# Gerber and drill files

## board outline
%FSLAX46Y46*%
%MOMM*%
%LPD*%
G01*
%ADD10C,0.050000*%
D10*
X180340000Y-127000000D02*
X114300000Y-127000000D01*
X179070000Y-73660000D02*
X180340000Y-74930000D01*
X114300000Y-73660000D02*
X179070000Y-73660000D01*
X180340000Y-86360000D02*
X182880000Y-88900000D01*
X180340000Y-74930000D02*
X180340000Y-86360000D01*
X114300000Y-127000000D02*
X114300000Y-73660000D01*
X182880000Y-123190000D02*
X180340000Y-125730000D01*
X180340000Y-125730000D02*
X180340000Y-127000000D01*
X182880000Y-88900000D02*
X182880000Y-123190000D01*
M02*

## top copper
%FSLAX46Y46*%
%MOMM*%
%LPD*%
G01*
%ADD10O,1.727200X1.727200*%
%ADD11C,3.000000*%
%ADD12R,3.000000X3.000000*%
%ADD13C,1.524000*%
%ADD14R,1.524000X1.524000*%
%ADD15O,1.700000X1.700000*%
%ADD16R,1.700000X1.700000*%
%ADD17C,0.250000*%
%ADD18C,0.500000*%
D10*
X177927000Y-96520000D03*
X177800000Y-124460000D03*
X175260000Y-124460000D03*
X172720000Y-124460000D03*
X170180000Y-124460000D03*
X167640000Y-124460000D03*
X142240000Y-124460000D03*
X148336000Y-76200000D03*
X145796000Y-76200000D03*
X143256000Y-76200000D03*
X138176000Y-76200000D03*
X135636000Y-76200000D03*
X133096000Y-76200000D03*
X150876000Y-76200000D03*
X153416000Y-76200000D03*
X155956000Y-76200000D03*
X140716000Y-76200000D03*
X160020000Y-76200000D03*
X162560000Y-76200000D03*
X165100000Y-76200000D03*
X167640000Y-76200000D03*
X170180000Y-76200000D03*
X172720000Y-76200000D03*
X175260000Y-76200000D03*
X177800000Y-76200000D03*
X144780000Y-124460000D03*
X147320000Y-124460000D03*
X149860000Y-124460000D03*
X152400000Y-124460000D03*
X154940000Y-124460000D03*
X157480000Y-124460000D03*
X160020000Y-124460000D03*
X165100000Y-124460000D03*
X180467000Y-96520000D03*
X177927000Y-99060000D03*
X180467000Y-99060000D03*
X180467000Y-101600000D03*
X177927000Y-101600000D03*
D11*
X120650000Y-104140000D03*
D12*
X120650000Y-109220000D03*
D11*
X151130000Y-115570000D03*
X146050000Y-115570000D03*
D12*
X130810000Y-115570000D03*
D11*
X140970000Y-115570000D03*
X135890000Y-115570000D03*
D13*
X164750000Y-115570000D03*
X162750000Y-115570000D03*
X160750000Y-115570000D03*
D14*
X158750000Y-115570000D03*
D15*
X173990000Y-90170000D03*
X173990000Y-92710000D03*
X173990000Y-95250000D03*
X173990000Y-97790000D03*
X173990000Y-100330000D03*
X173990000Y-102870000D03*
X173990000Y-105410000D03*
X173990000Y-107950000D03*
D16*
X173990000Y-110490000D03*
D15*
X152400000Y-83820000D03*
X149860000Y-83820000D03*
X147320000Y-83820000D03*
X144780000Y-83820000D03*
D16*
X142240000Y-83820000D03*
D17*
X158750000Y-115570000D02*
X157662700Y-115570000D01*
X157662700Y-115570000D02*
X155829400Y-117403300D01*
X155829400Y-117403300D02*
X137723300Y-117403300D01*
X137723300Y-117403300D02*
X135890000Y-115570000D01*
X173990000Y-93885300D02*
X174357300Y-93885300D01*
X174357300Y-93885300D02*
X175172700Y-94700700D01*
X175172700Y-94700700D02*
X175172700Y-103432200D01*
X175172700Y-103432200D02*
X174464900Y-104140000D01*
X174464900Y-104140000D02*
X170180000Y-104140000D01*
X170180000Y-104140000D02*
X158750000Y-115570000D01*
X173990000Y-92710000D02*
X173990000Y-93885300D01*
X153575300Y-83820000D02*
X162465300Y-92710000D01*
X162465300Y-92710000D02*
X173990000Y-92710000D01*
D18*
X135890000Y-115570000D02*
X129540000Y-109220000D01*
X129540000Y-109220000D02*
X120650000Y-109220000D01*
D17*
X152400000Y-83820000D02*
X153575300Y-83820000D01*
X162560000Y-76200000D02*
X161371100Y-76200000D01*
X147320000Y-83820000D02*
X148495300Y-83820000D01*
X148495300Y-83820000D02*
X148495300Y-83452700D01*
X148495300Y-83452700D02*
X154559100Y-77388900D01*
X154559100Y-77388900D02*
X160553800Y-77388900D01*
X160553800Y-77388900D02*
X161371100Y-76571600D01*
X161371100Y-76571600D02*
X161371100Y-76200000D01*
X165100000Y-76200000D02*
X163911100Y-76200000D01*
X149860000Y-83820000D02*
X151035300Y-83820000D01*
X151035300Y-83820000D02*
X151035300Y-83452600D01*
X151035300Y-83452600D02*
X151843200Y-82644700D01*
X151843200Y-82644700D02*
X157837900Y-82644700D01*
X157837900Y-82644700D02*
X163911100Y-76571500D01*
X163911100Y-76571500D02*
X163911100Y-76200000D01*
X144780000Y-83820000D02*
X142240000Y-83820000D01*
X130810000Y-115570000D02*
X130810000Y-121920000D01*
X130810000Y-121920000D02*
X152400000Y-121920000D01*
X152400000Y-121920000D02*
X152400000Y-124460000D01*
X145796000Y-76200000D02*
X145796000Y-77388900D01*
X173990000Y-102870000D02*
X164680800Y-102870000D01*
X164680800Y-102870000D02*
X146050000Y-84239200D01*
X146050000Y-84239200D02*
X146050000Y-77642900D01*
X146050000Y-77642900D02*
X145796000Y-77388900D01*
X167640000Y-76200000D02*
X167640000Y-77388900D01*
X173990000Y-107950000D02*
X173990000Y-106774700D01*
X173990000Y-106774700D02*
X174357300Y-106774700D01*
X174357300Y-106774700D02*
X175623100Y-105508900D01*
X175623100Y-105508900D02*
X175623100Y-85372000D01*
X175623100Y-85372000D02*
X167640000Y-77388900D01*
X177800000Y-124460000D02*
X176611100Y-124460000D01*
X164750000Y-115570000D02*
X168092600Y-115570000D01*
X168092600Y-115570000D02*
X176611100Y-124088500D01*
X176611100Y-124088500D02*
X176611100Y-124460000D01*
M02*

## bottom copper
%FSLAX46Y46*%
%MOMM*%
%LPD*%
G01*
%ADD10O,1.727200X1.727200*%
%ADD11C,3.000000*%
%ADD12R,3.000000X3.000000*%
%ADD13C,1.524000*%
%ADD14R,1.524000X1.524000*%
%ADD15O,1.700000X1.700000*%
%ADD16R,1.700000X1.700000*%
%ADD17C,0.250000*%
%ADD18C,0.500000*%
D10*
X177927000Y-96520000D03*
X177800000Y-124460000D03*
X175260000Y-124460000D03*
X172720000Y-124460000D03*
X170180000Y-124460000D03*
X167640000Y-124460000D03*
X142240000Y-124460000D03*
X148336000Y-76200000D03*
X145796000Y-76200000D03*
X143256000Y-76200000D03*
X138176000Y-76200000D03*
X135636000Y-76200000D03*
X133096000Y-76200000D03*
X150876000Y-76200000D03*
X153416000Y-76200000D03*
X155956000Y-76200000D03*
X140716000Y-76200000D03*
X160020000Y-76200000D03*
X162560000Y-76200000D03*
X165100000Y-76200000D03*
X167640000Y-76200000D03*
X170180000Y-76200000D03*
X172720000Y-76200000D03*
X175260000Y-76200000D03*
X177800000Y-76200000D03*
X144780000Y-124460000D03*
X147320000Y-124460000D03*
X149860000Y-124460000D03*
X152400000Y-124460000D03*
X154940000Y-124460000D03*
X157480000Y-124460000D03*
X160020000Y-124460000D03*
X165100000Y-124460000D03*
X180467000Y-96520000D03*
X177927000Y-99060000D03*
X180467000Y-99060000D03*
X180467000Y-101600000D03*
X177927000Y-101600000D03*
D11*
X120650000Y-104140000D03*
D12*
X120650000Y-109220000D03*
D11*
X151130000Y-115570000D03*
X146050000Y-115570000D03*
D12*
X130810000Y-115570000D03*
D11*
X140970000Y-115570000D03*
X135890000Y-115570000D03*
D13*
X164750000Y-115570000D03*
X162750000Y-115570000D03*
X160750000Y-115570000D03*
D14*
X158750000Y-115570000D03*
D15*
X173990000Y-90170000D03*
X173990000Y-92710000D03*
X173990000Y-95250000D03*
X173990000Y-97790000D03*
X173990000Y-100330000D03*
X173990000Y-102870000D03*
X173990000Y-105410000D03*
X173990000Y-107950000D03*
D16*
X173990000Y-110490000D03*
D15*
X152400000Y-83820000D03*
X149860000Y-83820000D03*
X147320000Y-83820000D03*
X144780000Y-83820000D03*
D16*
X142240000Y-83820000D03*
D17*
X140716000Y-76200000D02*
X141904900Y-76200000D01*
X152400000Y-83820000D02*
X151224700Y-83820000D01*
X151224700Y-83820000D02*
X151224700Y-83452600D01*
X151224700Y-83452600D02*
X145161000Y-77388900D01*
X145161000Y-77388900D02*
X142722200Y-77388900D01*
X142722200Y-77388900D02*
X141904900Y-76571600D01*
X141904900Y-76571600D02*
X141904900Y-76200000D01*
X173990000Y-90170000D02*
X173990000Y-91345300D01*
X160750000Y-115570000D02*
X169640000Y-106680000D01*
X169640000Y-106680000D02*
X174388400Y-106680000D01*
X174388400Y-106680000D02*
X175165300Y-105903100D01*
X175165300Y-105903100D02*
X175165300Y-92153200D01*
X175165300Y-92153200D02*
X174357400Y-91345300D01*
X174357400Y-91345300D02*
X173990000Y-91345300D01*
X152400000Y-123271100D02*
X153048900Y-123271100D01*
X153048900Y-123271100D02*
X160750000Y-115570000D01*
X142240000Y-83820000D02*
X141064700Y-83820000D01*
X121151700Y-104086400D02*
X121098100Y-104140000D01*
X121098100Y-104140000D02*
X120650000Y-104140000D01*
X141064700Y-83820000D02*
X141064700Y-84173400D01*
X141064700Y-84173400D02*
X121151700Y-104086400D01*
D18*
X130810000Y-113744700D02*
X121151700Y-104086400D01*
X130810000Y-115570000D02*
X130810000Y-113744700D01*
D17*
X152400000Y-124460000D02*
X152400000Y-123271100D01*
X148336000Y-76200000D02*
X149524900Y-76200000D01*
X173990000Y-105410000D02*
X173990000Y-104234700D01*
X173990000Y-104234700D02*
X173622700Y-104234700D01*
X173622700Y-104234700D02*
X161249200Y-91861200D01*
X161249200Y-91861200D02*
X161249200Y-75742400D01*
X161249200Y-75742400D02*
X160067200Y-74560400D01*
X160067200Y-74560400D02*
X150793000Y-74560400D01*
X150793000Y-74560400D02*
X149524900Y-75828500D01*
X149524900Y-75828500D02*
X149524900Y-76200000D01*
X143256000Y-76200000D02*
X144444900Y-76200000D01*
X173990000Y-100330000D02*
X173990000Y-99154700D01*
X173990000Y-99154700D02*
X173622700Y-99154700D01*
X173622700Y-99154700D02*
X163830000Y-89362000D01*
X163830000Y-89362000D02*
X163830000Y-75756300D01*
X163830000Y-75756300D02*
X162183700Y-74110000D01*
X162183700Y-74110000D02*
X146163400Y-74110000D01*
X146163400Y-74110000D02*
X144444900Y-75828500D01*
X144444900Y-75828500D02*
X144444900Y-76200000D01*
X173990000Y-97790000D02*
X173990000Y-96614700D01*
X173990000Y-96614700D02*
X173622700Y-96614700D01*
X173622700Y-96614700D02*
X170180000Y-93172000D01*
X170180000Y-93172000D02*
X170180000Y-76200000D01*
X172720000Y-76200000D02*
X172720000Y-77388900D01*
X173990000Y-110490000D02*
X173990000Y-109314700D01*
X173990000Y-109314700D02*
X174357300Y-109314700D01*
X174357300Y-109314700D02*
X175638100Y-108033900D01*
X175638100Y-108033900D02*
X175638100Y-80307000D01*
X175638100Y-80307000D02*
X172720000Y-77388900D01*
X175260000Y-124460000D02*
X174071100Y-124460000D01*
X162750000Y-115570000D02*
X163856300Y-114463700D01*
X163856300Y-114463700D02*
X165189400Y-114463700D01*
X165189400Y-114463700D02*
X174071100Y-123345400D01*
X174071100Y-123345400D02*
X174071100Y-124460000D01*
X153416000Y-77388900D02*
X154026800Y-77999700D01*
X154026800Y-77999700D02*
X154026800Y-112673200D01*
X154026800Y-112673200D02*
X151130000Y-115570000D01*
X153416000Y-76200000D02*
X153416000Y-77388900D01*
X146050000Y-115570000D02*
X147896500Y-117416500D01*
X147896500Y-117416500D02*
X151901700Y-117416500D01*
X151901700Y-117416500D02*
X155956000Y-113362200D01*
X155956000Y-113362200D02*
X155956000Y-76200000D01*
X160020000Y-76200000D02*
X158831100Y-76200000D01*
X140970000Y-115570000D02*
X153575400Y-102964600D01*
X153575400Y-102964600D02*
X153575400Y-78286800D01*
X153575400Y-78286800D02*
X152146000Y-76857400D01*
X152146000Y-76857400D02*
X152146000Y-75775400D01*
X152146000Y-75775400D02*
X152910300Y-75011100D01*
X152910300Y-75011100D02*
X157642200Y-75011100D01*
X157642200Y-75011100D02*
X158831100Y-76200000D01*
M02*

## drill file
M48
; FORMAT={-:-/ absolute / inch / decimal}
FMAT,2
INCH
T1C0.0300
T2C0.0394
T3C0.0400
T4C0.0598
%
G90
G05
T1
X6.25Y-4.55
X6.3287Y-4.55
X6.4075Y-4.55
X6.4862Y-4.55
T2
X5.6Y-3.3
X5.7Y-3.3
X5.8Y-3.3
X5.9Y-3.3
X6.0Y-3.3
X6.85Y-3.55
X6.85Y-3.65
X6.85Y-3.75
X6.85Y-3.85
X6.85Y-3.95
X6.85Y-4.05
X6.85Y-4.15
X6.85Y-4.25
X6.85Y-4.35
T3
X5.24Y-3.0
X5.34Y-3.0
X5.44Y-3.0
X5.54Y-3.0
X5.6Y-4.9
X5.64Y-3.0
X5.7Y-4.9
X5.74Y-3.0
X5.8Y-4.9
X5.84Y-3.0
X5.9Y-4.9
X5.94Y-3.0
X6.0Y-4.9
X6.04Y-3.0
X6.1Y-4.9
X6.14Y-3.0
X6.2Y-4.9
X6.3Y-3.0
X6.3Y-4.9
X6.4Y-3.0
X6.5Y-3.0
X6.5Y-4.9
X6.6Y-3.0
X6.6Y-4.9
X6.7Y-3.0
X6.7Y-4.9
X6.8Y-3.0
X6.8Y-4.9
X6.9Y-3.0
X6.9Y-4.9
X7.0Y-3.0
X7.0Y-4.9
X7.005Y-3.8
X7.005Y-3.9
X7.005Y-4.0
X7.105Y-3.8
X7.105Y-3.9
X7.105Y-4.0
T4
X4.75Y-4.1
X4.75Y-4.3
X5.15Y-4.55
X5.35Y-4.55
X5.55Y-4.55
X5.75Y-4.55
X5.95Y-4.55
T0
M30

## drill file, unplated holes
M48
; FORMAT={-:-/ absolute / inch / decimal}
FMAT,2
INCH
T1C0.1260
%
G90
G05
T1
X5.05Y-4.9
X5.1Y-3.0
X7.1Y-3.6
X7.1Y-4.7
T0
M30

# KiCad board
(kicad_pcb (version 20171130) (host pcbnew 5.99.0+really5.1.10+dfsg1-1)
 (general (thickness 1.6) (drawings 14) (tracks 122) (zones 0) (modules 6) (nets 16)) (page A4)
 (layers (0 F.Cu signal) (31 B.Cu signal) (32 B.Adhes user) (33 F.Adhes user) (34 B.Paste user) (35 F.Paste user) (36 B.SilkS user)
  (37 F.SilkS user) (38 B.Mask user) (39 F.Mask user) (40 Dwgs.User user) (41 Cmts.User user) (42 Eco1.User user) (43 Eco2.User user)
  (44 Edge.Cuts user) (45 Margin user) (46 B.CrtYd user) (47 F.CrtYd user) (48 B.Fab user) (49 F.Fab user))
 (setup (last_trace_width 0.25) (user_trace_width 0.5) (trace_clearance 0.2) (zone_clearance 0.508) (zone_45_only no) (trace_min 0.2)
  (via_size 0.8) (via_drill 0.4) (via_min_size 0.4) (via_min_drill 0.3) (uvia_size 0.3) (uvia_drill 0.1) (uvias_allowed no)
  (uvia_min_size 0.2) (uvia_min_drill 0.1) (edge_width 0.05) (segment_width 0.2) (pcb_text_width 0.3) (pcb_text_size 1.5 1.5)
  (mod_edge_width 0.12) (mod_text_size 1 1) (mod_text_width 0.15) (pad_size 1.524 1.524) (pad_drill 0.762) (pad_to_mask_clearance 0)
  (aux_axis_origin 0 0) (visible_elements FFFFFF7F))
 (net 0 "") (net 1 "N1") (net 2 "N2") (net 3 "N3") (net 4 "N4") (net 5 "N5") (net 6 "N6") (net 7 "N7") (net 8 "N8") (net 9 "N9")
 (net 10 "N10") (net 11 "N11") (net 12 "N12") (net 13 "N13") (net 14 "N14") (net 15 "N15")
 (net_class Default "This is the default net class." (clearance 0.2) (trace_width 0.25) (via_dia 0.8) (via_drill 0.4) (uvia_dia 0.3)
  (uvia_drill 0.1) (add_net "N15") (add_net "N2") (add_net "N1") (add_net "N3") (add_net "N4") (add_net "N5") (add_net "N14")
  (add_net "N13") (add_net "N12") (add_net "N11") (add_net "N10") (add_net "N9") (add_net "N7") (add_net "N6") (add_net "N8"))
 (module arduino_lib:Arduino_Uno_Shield (layer F.Cu) (at 114.3 127)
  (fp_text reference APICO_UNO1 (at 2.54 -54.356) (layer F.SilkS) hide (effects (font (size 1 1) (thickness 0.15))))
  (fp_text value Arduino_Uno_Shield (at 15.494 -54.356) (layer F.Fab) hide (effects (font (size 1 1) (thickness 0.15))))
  (pad MISO thru_hole oval (at 63.627 -30.48) (size 1.7272 1.7272) (drill 1.016) (layers *.Cu *.Mask))
  (pad A5 thru_hole oval (at 63.5 -2.54) (size 1.7272 1.7272) (drill 1.016) (layers *.Cu *.Mask) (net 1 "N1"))
  (pad A4 thru_hole oval (at 60.96 -2.54) (size 1.7272 1.7272) (drill 1.016) (layers *.Cu *.Mask) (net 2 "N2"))
  (pad A3 thru_hole oval (at 58.42 -2.54) (size 1.7272 1.7272) (drill 1.016) (layers *.Cu *.Mask))
  (pad A2 thru_hole oval (at 55.88 -2.54) (size 1.7272 1.7272) (drill 1.016) (layers *.Cu *.Mask))
  (pad A1 thru_hole oval (at 53.34 -2.54) (size 1.7272 1.7272) (drill 1.016) (layers *.Cu *.Mask))
  (pad "" thru_hole oval (at 27.94 -2.54) (size 1.7272 1.7272) (drill 1.016) (layers *.Cu *.Mask))
  (pad D11 thru_hole oval (at 34.036 -50.8) (size 1.7272 1.7272) (drill 1.016) (layers *.Cu *.Mask) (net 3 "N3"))
  (pad D12 thru_hole oval (at 31.496 -50.8) (size 1.7272 1.7272) (drill 1.016) (layers *.Cu *.Mask) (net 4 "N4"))
  (pad D13 thru_hole oval (at 28.956 -50.8) (size 1.7272 1.7272) (drill 1.016) (layers *.Cu *.Mask) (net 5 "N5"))
  (pad AREF thru_hole oval (at 23.876 -50.8) (size 1.7272 1.7272) (drill 1.016) (layers *.Cu *.Mask))
  (pad SDA thru_hole oval (at 21.336 -50.8) (size 1.7272 1.7272) (drill 1.016) (layers *.Cu *.Mask))
  (pad SCL thru_hole oval (at 18.796 -50.8) (size 1.7272 1.7272) (drill 1.016) (layers *.Cu *.Mask))
  (pad "" np_thru_hole circle (at 13.97 -2.54) (size 3.2 3.2) (drill 3.2) (layers *.Cu *.Mask))
  (pad "" np_thru_hole circle (at 15.24 -50.8) (size 3.2 3.2) (drill 3.2) (layers *.Cu *.Mask))
  (pad "" np_thru_hole circle (at 66.04 -35.56) (size 3.2 3.2) (drill 3.2) (layers *.Cu *.Mask))
  (pad "" np_thru_hole circle (at 66.04 -7.62) (size 3.2 3.2) (drill 3.2) (layers *.Cu *.Mask))
  (pad D10 thru_hole oval (at 36.576 -50.8) (size 1.7272 1.7272) (drill 1.016) (layers *.Cu *.Mask))
  (pad D9 thru_hole oval (at 39.116 -50.8) (size 1.7272 1.7272) (drill 1.016) (layers *.Cu *.Mask) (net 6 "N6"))
  (pad D8 thru_hole oval (at 41.656 -50.8) (size 1.7272 1.7272) (drill 1.016) (layers *.Cu *.Mask) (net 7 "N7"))
  (pad GND1 thru_hole oval (at 26.416 -50.8) (size 1.7272 1.7272) (drill 1.016) (layers *.Cu *.Mask) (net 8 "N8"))
  (pad D7 thru_hole oval (at 45.72 -50.8) (size 1.7272 1.7272) (drill 1.016) (layers *.Cu *.Mask) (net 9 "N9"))
  (pad D6 thru_hole oval (at 48.26 -50.8) (size 1.7272 1.7272) (drill 1.016) (layers *.Cu *.Mask) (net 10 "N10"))
  (pad D5 thru_hole oval (at 50.8 -50.8) (size 1.7272 1.7272) (drill 1.016) (layers *.Cu *.Mask) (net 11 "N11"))
  (pad D4 thru_hole oval (at 53.34 -50.8) (size 1.7272 1.7272) (drill 1.016) (layers *.Cu *.Mask) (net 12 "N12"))
  (pad D3 thru_hole oval (at 55.88 -50.8) (size 1.7272 1.7272) (drill 1.016) (layers *.Cu *.Mask) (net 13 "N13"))
  (pad D2 thru_hole oval (at 58.42 -50.8) (size 1.7272 1.7272) (drill 1.016) (layers *.Cu *.Mask) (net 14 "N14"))
  (pad D1 thru_hole oval (at 60.96 -50.8) (size 1.7272 1.7272) (drill 1.016) (layers *.Cu *.Mask))
  (pad D0 thru_hole oval (at 63.5 -50.8) (size 1.7272 1.7272) (drill 1.016) (layers *.Cu *.Mask))
  (pad IORF thru_hole oval (at 30.48 -2.54) (size 1.7272 1.7272) (drill 1.016) (layers *.Cu *.Mask))
  (pad RST1 thru_hole oval (at 33.02 -2.54) (size 1.7272 1.7272) (drill 1.016) (layers *.Cu *.Mask))
  (pad 3V3 thru_hole oval (at 35.56 -2.54) (size 1.7272 1.7272) (drill 1.016) (layers *.Cu *.Mask))
  (pad 5V1 thru_hole oval (at 38.1 -2.54) (size 1.7272 1.7272) (drill 1.016) (layers *.Cu *.Mask) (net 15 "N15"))
  (pad GND2 thru_hole oval (at 40.64 -2.54) (size 1.7272 1.7272) (drill 1.016) (layers *.Cu *.Mask))
  (pad GND3 thru_hole oval (at 43.18 -2.54) (size 1.7272 1.7272) (drill 1.016) (layers *.Cu *.Mask))
  (pad VIN thru_hole oval (at 45.72 -2.54) (size 1.7272 1.7272) (drill 1.016) (layers *.Cu *.Mask))
  (pad A0 thru_hole oval (at 50.8 -2.54) (size 1.7272 1.7272) (drill 1.016) (layers *.Cu *.Mask))
  (pad 5V2 thru_hole oval (at 66.167 -30.48) (size 1.7272 1.7272) (drill 1.016) (layers *.Cu *.Mask))
  (pad SCK thru_hole oval (at 63.627 -27.94) (size 1.7272 1.7272) (drill 1.016) (layers *.Cu *.Mask))
  (pad MOSI thru_hole oval (at 66.167 -27.94) (size 1.7272 1.7272) (drill 1.016) (layers *.Cu *.Mask))
  (pad GND4 thru_hole oval (at 66.167 -25.4) (size 1.7272 1.7272) (drill 1.016) (layers *.Cu *.Mask))
  (pad RST2 thru_hole oval (at 63.627 -25.4) (size 1.7272 1.7272) (drill 1.016) (layers *.Cu *.Mask)))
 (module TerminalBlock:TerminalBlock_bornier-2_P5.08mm (layer F.Cu) (at 120.65 109.22 90)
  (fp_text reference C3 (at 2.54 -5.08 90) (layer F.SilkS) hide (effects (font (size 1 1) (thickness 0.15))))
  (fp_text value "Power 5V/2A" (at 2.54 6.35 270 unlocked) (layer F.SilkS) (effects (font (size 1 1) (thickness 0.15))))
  (pad 2 thru_hole circle (at 5.08 0 90) (size 3 3) (drill 1.52) (layers *.Cu *.Mask) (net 15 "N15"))
  (pad 1 thru_hole rect (at 0 0 90) (size 3 3) (drill 1.52) (layers *.Cu *.Mask) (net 8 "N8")))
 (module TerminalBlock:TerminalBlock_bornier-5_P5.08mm (layer F.Cu) (at 130.81 115.57)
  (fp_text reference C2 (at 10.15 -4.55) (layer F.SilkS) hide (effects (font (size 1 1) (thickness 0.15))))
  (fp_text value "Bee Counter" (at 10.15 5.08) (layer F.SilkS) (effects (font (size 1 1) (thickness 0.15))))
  (pad 5 thru_hole circle (at 20.32 0) (size 3 3) (drill 1.52) (layers *.Cu *.Mask) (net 6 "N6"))
  (pad 4 thru_hole circle (at 15.24 0) (size 3 3) (drill 1.52) (layers *.Cu *.Mask) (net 7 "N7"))
  (pad 1 thru_hole rect (at 0 0) (size 3 3) (drill 1.52) (layers *.Cu *.Mask) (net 15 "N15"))
  (pad 3 thru_hole circle (at 10.16 0) (size 3 3) (drill 1.52) (layers *.Cu *.Mask) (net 9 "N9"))
  (pad 2 thru_hole circle (at 5.08 0) (size 3 3) (drill 1.52) (layers *.Cu *.Mask) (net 8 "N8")))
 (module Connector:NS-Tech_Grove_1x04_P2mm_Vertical (layer F.Cu) (at 158.75 115.57 90)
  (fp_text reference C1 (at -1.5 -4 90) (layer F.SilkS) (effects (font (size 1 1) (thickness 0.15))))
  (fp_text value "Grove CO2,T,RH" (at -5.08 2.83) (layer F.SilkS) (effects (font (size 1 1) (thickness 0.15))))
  (pad 4 thru_hole circle (at 0 6 90) (size 1.524 1.524) (drill 0.762) (layers *.Cu *.Mask) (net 1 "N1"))
  (pad 3 thru_hole circle (at 0 4 90) (size 1.524 1.524) (drill 0.762) (layers *.Cu *.Mask) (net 2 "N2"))
  (pad 2 thru_hole circle (at 0 2 90) (size 1.524 1.524) (drill 0.762) (layers *.Cu *.Mask) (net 15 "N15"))
  (pad 1 thru_hole rect (at 0 0 90) (size 1.524 1.524) (drill 0.762) (layers *.Cu *.Mask) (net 8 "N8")))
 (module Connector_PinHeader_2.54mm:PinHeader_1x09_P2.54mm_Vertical (layer F.Cu) (at 173.99 110.49 180)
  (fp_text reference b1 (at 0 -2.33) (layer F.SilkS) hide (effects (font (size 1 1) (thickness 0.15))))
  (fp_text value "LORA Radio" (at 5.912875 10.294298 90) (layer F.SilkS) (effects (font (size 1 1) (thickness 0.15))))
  (pad 9 thru_hole oval (at 0 20.32 180) (size 1.7 1.7) (drill 1) (layers *.Cu *.Mask) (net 15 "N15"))
  (pad 8 thru_hole oval (at 0 17.78 180) (size 1.7 1.7) (drill 1) (layers *.Cu *.Mask) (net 8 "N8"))
  (pad 7 thru_hole oval (at 0 15.24 180) (size 1.7 1.7) (drill 1) (layers *.Cu *.Mask))
  (pad 6 thru_hole oval (at 0 12.7 180) (size 1.7 1.7) (drill 1) (layers *.Cu *.Mask) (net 13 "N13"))
  (pad 5 thru_hole oval (at 0 10.16 180) (size 1.7 1.7) (drill 1) (layers *.Cu *.Mask) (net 5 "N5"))
  (pad 4 thru_hole oval (at 0 7.62 180) (size 1.7 1.7) (drill 1) (layers *.Cu *.Mask) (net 4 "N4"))
  (pad 3 thru_hole oval (at 0 5.08 180) (size 1.7 1.7) (drill 1) (layers *.Cu *.Mask) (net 3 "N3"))
  (pad 2 thru_hole oval (at 0 2.54 180) (size 1.7 1.7) (drill 1) (layers *.Cu *.Mask) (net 12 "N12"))
  (pad 1 thru_hole rect (at 0 0 180) (size 1.7 1.7) (drill 1) (layers *.Cu *.Mask) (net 14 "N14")))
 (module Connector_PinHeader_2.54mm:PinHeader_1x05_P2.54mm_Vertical (layer F.Cu) (at 142.24 83.82 90)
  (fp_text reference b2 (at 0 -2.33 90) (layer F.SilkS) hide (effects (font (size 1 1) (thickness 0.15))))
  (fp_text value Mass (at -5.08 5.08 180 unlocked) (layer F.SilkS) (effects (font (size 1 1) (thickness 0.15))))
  (pad 5 thru_hole oval (at 0 10.16 90) (size 1.7 1.7) (drill 1) (layers *.Cu *.Mask) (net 8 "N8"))
  (pad 4 thru_hole oval (at 0 7.62 90) (size 1.7 1.7) (drill 1) (layers *.Cu *.Mask) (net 11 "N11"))
  (pad 3 thru_hole oval (at 0 5.08 90) (size 1.7 1.7) (drill 1) (layers *.Cu *.Mask) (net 10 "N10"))
  (pad 2 thru_hole oval (at 0 2.54 90) (size 1.7 1.7) (drill 1) (layers *.Cu *.Mask) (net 15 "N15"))
  (pad 1 thru_hole rect (at 0 0 90) (size 1.7 1.7) (drill 1) (layers *.Cu *.Mask) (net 15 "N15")))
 (gr_line (start 180.34 127) (end 114.3 127) (layer Edge.Cuts) (width 0.05))
 (gr_line (start 179.07 73.66) (end 180.34 74.93) (layer Edge.Cuts) (width 0.05))
 (gr_line (start 114.3 73.66) (end 179.07 73.66) (layer Edge.Cuts) (width 0.05))
 (gr_line (start 180.34 86.36) (end 182.88 88.9) (layer Edge.Cuts) (width 0.05))
 (gr_line (start 180.34 74.93) (end 180.34 86.36) (layer Edge.Cuts) (width 0.05))
 (gr_line (start 114.3 127) (end 114.3 73.66) (layer Edge.Cuts) (width 0.05))
 (gr_line (start 182.88 123.19) (end 180.34 125.73) (layer Edge.Cuts) (width 0.05))
 (gr_line (start 180.34 125.73) (end 180.34 127) (layer Edge.Cuts) (width 0.05))
 (gr_line (start 182.88 88.9) (end 182.88 123.19) (layer Edge.Cuts) (width 0.05))
 (segment (start 158.75 115.57) (end 157.6627 115.57) (width 0.25) (layer F.Cu) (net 8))
 (segment (start 157.6627 115.57) (end 155.8294 117.4033) (width 0.25) (layer F.Cu) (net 8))
 (segment (start 155.8294 117.4033) (end 137.7233 117.4033) (width 0.25) (layer F.Cu) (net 8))
 (segment (start 137.7233 117.4033) (end 135.89 115.57) (width 0.25) (layer F.Cu) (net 8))
 (segment (start 173.99 93.8853) (end 174.3573 93.8853) (width 0.25) (layer F.Cu) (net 8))
 (segment (start 174.3573 93.8853) (end 175.1727 94.7007) (width 0.25) (layer F.Cu) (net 8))
 (segment (start 175.1727 94.7007) (end 175.1727 103.4322) (width 0.25) (layer F.Cu) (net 8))
 (segment (start 175.1727 103.4322) (end 174.4649 104.14) (width 0.25) (layer F.Cu) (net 8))
 (segment (start 174.4649 104.14) (end 170.18 104.14) (width 0.25) (layer F.Cu) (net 8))
 (segment (start 170.18 104.14) (end 158.75 115.57) (width 0.25) (layer F.Cu) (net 8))
 (segment (start 173.99 92.71) (end 173.99 93.8853) (width 0.25) (layer F.Cu) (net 8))
 (segment (start 153.5753 83.82) (end 162.4653 92.71) (width 0.25) (layer F.Cu) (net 8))
 (segment (start 162.4653 92.71) (end 173.99 92.71) (width 0.25) (layer F.Cu) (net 8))
 (segment (start 140.716 76.2) (end 141.9049 76.2) (width 0.25) (layer B.Cu) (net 8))
 (segment (start 152.4 83.82) (end 151.2247 83.82) (width 0.25) (layer B.Cu) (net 8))
 (segment (start 151.2247 83.82) (end 151.2247 83.4526) (width 0.25) (layer B.Cu) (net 8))
 (segment (start 151.2247 83.4526) (end 145.161 77.3889) (width 0.25) (layer B.Cu) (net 8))
 (segment (start 145.161 77.3889) (end 142.7222 77.3889) (width 0.25) (layer B.Cu) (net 8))
 (segment (start 142.7222 77.3889) (end 141.9049 76.5716) (width 0.25) (layer B.Cu) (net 8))
 (segment (start 141.9049 76.5716) (end 141.9049 76.2) (width 0.25) (layer B.Cu) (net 8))
 (segment (start 135.89 115.57) (end 129.54 109.22) (width 0.5) (layer F.Cu) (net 8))
 (segment (start 129.54 109.22) (end 120.65 109.22) (width 0.5) (layer F.Cu) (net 8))
 (segment (start 152.4 83.82) (end 153.5753 83.82) (width 0.25) (layer F.Cu) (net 8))
 (segment (start 162.56 76.2) (end 161.3711 76.2) (width 0.25) (layer F.Cu) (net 10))
 (segment (start 147.32 83.82) (end 148.4953 83.82) (width 0.25) (layer F.Cu) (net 10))
 (segment (start 148.4953 83.82) (end 148.4953 83.4527) (width 0.25) (layer F.Cu) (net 10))
 (segment (start 148.4953 83.4527) (end 154.5591 77.3889) (width 0.25) (layer F.Cu) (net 10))
 (segment (start 154.5591 77.3889) (end 160.5538 77.3889) (width 0.25) (layer F.Cu) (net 10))
 (segment (start 160.5538 77.3889) (end 161.3711 76.5716) (width 0.25) (layer F.Cu) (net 10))
 (segment (start 161.3711 76.5716) (end 161.3711 76.2) (width 0.25) (layer F.Cu) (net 10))
 (segment (start 165.1 76.2) (end 163.9111 76.2) (width 0.25) (layer F.Cu) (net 11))
 (segment (start 149.86 83.82) (end 151.0353 83.82) (width 0.25) (layer F.Cu) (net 11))
 (segment (start 151.0353 83.82) (end 151.0353 83.4526) (width 0.25) (layer F.Cu) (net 11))
 (segment (start 151.0353 83.4526) (end 151.8432 82.6447) (width 0.25) (layer F.Cu) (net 11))
 (segment (start 151.8432 82.6447) (end 157.8379 82.6447) (width 0.25) (layer F.Cu) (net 11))
 (segment (start 157.8379 82.6447) (end 163.9111 76.5715) (width 0.25) (layer F.Cu) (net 11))
 (segment (start 163.9111 76.5715) (end 163.9111 76.2) (width 0.25) (layer F.Cu) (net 11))
 (segment (start 173.99 90.17) (end 173.99 91.3453) (width 0.25) (layer B.Cu) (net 15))
 (segment (start 160.75 115.57) (end 169.64 106.68) (width 0.25) (layer B.Cu) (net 15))
 (segment (start 169.64 106.68) (end 174.3884 106.68) (width 0.25) (layer B.Cu) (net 15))
 (segment (start 174.3884 106.68) (end 175.1653 105.9031) (width 0.25) (layer B.Cu) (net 15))
 (segment (start 175.1653 105.9031) (end 175.1653 92.1532) (width 0.25) (layer B.Cu) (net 15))
 (segment (start 175.1653 92.1532) (end 174.3574 91.3453) (width 0.25) (layer B.Cu) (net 15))
 (segment (start 174.3574 91.3453) (end 173.99 91.3453) (width 0.25) (layer B.Cu) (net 15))
 (segment (start 152.4 123.2711) (end 153.0489 123.2711) (width 0.25) (layer B.Cu) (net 15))
 (segment (start 153.0489 123.2711) (end 160.75 115.57) (width 0.25) (layer B.Cu) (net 15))
 (segment (start 142.24 83.82) (end 141.0647 83.82) (width 0.25) (layer B.Cu) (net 15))
 (segment (start 121.1517 104.0864) (end 121.0981 104.14) (width 0.25) (layer B.Cu) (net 15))
 (segment (start 121.0981 104.14) (end 120.65 104.14) (width 0.25) (layer B.Cu) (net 15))
 (segment (start 141.0647 83.82) (end 141.0647 84.1734) (width 0.25) (layer B.Cu) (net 15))
 (segment (start 141.0647 84.1734) (end 121.1517 104.0864) (width 0.25) (layer B.Cu) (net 15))
 (segment (start 130.81 113.7447) (end 121.1517 104.0864) (width 0.5) (layer B.Cu) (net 15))
 (segment (start 130.81 115.57) (end 130.81 113.7447) (width 0.5) (layer B.Cu) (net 15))
 (segment (start 144.78 83.82) (end 142.24 83.82) (width 0.25) (layer F.Cu) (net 15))
 (segment (start 152.4 124.46) (end 152.4 123.2711) (width 0.25) (layer B.Cu) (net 15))
 (segment (start 130.81 115.57) (end 130.81 121.92) (width 0.25) (layer F.Cu) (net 15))
 (segment (start 130.81 121.92) (end 152.4 121.92) (width 0.25) (layer F.Cu) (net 15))
 (segment (start 152.4 121.92) (end 152.4 124.46) (width 0.25) (layer F.Cu) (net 15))
 (segment (start 148.336 76.2) (end 149.5249 76.2) (width 0.25) (layer B.Cu) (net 3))
 (segment (start 173.99 105.41) (end 173.99 104.2347) (width 0.25) (layer B.Cu) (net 3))
 (segment (start 173.99 104.2347) (end 173.6227 104.2347) (width 0.25) (layer B.Cu) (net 3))
 (segment (start 173.6227 104.2347) (end 161.2492 91.8612) (width 0.25) (layer B.Cu) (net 3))
 (segment (start 161.2492 91.8612) (end 161.2492 75.7424) (width 0.25) (layer B.Cu) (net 3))
 (segment (start 161.2492 75.7424) (end 160.0672 74.5604) (width 0.25) (layer B.Cu) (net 3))
 (segment (start 160.0672 74.5604) (end 150.793 74.5604) (width 0.25) (layer B.Cu) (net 3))
 (segment (start 150.793 74.5604) (end 149.5249 75.8285) (width 0.25) (layer B.Cu) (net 3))
 (segment (start 149.5249 75.8285) (end 149.5249 76.2) (width 0.25) (layer B.Cu) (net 3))
 (segment (start 145.796 76.2) (end 145.796 77.3889) (width 0.25) (layer F.Cu) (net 4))
 (segment (start 173.99 102.87) (end 164.6808 102.87) (width 0.25) (layer F.Cu) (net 4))
 (segment (start 164.6808 102.87) (end 146.05 84.2392) (width 0.25) (layer F.Cu) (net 4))
 (segment (start 146.05 84.2392) (end 146.05 77.6429) (width 0.25) (layer F.Cu) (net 4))
 (segment (start 146.05 77.6429) (end 145.796 77.3889) (width 0.25) (layer F.Cu) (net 4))
 (segment (start 143.256 76.2) (end 144.4449 76.2) (width 0.25) (layer B.Cu) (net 5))
 (segment (start 173.99 100.33) (end 173.99 99.1547) (width 0.25) (layer B.Cu) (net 5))
 (segment (start 173.99 99.1547) (end 173.6227 99.1547) (width 0.25) (layer B.Cu) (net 5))
 (segment (start 173.6227 99.1547) (end 163.83 89.362) (width 0.25) (layer B.Cu) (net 5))
 (segment (start 163.83 89.362) (end 163.83 75.7563) (width 0.25) (layer B.Cu) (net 5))
 (segment (start 163.83 75.7563) (end 162.1837 74.11) (width 0.25) (layer B.Cu) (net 5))
 (segment (start 162.1837 74.11) (end 146.1634 74.11) (width 0.25) (layer B.Cu) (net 5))
 (segment (start 146.1634 74.11) (end 144.4449 75.8285) (width 0.25) (layer B.Cu) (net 5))
 (segment (start 144.4449 75.8285) (end 144.4449 76.2) (width 0.25) (layer B.Cu) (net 5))
 (segment (start 167.64 76.2) (end 167.64 77.3889) (width 0.25) (layer F.Cu) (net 12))
 (segment (start 173.99 107.95) (end 173.99 106.7747) (width 0.25) (layer F.Cu) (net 12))
 (segment (start 173.99 106.7747) (end 174.3573 106.7747) (width 0.25) (layer F.Cu) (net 12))
 (segment (start 174.3573 106.7747) (end 175.6231 105.5089) (width 0.25) (layer F.Cu) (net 12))
 (segment (start 175.6231 105.5089) (end 175.6231 85.372) (width 0.25) (layer F.Cu) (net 12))
 (segment (start 175.6231 85.372) (end 167.64 77.3889) (width 0.25) (layer F.Cu) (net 12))
 (segment (start 173.99 97.79) (end 173.99 96.6147) (width 0.25) (layer B.Cu) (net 13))
 (segment (start 173.99 96.6147) (end 173.6227 96.6147) (width 0.25) (layer B.Cu) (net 13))
 (segment (start 173.6227 96.6147) (end 170.18 93.172) (width 0.25) (layer B.Cu) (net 13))
 (segment (start 170.18 93.172) (end 170.18 76.2) (width 0.25) (layer B.Cu) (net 13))
 (segment (start 172.72 76.2) (end 172.72 77.3889) (width 0.25) (layer B.Cu) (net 14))
 (segment (start 173.99 110.49) (end 173.99 109.3147) (width 0.25) (layer B.Cu) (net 14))
 (segment (start 173.99 109.3147) (end 174.3573 109.3147) (width 0.25) (layer B.Cu) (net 14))
 (segment (start 174.3573 109.3147) (end 175.6381 108.0339) (width 0.25) (layer B.Cu) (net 14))
 (segment (start 175.6381 108.0339) (end 175.6381 80.307) (width 0.25) (layer B.Cu) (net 14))
 (segment (start 175.6381 80.307) (end 172.72 77.3889) (width 0.25) (layer B.Cu) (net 14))
 (segment (start 177.8 124.46) (end 176.6111 124.46) (width 0.25) (layer F.Cu) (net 1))
 (segment (start 164.75 115.57) (end 168.0926 115.57) (width 0.25) (layer F.Cu) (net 1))
 (segment (start 168.0926 115.57) (end 176.6111 124.0885) (width 0.25) (layer F.Cu) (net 1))
 (segment (start 176.6111 124.0885) (end 176.6111 124.46) (width 0.25) (layer F.Cu) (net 1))
 (segment (start 175.26 124.46) (end 174.0711 124.46) (width 0.25) (layer B.Cu) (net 2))
 (segment (start 162.75 115.57) (end 163.8563 114.4637) (width 0.25) (layer B.Cu) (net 2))
 (segment (start 163.8563 114.4637) (end 165.1894 114.4637) (width 0.25) (layer B.Cu) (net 2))
 (segment (start 165.1894 114.4637) (end 174.0711 123.3454) (width 0.25) (layer B.Cu) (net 2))
 (segment (start 174.0711 123.3454) (end 174.0711 124.46) (width 0.25) (layer B.Cu) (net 2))
 (segment (start 153.416 77.3889) (end 154.0268 77.9997) (width 0.25) (layer B.Cu) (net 6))
 (segment (start 154.0268 77.9997) (end 154.0268 112.6732) (width 0.25) (layer B.Cu) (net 6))
 (segment (start 154.0268 112.6732) (end 151.13 115.57) (width 0.25) (layer B.Cu) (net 6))
 (segment (start 153.416 76.2) (end 153.416 77.3889) (width 0.25) (layer B.Cu) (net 6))
 (segment (start 146.05 115.57) (end 147.8965 117.4165) (width 0.25) (layer B.Cu) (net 7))
 (segment (start 147.8965 117.4165) (end 151.9017 117.4165) (width 0.25) (layer B.Cu) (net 7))
 (segment (start 151.9017 117.4165) (end 155.956 113.3622) (width 0.25) (layer B.Cu) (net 7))
 (segment (start 155.956 113.3622) (end 155.956 76.2) (width 0.25) (layer B.Cu) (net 7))
 (segment (start 160.02 76.2) (end 158.8311 76.2) (width 0.25) (layer B.Cu) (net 9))
 (segment (start 140.97 115.57) (end 153.5754 102.9646) (width 0.25) (layer B.Cu) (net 9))
 (segment (start 153.5754 102.9646) (end 153.5754 78.2868) (width 0.25) (layer B.Cu) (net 9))
 (segment (start 153.5754 78.2868) (end 152.146 76.8574) (width 0.25) (layer B.Cu) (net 9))
 (segment (start 152.146 76.8574) (end 152.146 75.7754) (width 0.25) (layer B.Cu) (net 9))
 (segment (start 152.146 75.7754) (end 152.9103 75.0111) (width 0.25) (layer B.Cu) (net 9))
 (segment (start 152.9103 75.0111) (end 157.6422 75.0111) (width 0.25) (layer B.Cu) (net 9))
 (segment (start 157.6422 75.0111) (end 158.8311 76.2) (width 0.25) (layer B.Cu) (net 9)))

